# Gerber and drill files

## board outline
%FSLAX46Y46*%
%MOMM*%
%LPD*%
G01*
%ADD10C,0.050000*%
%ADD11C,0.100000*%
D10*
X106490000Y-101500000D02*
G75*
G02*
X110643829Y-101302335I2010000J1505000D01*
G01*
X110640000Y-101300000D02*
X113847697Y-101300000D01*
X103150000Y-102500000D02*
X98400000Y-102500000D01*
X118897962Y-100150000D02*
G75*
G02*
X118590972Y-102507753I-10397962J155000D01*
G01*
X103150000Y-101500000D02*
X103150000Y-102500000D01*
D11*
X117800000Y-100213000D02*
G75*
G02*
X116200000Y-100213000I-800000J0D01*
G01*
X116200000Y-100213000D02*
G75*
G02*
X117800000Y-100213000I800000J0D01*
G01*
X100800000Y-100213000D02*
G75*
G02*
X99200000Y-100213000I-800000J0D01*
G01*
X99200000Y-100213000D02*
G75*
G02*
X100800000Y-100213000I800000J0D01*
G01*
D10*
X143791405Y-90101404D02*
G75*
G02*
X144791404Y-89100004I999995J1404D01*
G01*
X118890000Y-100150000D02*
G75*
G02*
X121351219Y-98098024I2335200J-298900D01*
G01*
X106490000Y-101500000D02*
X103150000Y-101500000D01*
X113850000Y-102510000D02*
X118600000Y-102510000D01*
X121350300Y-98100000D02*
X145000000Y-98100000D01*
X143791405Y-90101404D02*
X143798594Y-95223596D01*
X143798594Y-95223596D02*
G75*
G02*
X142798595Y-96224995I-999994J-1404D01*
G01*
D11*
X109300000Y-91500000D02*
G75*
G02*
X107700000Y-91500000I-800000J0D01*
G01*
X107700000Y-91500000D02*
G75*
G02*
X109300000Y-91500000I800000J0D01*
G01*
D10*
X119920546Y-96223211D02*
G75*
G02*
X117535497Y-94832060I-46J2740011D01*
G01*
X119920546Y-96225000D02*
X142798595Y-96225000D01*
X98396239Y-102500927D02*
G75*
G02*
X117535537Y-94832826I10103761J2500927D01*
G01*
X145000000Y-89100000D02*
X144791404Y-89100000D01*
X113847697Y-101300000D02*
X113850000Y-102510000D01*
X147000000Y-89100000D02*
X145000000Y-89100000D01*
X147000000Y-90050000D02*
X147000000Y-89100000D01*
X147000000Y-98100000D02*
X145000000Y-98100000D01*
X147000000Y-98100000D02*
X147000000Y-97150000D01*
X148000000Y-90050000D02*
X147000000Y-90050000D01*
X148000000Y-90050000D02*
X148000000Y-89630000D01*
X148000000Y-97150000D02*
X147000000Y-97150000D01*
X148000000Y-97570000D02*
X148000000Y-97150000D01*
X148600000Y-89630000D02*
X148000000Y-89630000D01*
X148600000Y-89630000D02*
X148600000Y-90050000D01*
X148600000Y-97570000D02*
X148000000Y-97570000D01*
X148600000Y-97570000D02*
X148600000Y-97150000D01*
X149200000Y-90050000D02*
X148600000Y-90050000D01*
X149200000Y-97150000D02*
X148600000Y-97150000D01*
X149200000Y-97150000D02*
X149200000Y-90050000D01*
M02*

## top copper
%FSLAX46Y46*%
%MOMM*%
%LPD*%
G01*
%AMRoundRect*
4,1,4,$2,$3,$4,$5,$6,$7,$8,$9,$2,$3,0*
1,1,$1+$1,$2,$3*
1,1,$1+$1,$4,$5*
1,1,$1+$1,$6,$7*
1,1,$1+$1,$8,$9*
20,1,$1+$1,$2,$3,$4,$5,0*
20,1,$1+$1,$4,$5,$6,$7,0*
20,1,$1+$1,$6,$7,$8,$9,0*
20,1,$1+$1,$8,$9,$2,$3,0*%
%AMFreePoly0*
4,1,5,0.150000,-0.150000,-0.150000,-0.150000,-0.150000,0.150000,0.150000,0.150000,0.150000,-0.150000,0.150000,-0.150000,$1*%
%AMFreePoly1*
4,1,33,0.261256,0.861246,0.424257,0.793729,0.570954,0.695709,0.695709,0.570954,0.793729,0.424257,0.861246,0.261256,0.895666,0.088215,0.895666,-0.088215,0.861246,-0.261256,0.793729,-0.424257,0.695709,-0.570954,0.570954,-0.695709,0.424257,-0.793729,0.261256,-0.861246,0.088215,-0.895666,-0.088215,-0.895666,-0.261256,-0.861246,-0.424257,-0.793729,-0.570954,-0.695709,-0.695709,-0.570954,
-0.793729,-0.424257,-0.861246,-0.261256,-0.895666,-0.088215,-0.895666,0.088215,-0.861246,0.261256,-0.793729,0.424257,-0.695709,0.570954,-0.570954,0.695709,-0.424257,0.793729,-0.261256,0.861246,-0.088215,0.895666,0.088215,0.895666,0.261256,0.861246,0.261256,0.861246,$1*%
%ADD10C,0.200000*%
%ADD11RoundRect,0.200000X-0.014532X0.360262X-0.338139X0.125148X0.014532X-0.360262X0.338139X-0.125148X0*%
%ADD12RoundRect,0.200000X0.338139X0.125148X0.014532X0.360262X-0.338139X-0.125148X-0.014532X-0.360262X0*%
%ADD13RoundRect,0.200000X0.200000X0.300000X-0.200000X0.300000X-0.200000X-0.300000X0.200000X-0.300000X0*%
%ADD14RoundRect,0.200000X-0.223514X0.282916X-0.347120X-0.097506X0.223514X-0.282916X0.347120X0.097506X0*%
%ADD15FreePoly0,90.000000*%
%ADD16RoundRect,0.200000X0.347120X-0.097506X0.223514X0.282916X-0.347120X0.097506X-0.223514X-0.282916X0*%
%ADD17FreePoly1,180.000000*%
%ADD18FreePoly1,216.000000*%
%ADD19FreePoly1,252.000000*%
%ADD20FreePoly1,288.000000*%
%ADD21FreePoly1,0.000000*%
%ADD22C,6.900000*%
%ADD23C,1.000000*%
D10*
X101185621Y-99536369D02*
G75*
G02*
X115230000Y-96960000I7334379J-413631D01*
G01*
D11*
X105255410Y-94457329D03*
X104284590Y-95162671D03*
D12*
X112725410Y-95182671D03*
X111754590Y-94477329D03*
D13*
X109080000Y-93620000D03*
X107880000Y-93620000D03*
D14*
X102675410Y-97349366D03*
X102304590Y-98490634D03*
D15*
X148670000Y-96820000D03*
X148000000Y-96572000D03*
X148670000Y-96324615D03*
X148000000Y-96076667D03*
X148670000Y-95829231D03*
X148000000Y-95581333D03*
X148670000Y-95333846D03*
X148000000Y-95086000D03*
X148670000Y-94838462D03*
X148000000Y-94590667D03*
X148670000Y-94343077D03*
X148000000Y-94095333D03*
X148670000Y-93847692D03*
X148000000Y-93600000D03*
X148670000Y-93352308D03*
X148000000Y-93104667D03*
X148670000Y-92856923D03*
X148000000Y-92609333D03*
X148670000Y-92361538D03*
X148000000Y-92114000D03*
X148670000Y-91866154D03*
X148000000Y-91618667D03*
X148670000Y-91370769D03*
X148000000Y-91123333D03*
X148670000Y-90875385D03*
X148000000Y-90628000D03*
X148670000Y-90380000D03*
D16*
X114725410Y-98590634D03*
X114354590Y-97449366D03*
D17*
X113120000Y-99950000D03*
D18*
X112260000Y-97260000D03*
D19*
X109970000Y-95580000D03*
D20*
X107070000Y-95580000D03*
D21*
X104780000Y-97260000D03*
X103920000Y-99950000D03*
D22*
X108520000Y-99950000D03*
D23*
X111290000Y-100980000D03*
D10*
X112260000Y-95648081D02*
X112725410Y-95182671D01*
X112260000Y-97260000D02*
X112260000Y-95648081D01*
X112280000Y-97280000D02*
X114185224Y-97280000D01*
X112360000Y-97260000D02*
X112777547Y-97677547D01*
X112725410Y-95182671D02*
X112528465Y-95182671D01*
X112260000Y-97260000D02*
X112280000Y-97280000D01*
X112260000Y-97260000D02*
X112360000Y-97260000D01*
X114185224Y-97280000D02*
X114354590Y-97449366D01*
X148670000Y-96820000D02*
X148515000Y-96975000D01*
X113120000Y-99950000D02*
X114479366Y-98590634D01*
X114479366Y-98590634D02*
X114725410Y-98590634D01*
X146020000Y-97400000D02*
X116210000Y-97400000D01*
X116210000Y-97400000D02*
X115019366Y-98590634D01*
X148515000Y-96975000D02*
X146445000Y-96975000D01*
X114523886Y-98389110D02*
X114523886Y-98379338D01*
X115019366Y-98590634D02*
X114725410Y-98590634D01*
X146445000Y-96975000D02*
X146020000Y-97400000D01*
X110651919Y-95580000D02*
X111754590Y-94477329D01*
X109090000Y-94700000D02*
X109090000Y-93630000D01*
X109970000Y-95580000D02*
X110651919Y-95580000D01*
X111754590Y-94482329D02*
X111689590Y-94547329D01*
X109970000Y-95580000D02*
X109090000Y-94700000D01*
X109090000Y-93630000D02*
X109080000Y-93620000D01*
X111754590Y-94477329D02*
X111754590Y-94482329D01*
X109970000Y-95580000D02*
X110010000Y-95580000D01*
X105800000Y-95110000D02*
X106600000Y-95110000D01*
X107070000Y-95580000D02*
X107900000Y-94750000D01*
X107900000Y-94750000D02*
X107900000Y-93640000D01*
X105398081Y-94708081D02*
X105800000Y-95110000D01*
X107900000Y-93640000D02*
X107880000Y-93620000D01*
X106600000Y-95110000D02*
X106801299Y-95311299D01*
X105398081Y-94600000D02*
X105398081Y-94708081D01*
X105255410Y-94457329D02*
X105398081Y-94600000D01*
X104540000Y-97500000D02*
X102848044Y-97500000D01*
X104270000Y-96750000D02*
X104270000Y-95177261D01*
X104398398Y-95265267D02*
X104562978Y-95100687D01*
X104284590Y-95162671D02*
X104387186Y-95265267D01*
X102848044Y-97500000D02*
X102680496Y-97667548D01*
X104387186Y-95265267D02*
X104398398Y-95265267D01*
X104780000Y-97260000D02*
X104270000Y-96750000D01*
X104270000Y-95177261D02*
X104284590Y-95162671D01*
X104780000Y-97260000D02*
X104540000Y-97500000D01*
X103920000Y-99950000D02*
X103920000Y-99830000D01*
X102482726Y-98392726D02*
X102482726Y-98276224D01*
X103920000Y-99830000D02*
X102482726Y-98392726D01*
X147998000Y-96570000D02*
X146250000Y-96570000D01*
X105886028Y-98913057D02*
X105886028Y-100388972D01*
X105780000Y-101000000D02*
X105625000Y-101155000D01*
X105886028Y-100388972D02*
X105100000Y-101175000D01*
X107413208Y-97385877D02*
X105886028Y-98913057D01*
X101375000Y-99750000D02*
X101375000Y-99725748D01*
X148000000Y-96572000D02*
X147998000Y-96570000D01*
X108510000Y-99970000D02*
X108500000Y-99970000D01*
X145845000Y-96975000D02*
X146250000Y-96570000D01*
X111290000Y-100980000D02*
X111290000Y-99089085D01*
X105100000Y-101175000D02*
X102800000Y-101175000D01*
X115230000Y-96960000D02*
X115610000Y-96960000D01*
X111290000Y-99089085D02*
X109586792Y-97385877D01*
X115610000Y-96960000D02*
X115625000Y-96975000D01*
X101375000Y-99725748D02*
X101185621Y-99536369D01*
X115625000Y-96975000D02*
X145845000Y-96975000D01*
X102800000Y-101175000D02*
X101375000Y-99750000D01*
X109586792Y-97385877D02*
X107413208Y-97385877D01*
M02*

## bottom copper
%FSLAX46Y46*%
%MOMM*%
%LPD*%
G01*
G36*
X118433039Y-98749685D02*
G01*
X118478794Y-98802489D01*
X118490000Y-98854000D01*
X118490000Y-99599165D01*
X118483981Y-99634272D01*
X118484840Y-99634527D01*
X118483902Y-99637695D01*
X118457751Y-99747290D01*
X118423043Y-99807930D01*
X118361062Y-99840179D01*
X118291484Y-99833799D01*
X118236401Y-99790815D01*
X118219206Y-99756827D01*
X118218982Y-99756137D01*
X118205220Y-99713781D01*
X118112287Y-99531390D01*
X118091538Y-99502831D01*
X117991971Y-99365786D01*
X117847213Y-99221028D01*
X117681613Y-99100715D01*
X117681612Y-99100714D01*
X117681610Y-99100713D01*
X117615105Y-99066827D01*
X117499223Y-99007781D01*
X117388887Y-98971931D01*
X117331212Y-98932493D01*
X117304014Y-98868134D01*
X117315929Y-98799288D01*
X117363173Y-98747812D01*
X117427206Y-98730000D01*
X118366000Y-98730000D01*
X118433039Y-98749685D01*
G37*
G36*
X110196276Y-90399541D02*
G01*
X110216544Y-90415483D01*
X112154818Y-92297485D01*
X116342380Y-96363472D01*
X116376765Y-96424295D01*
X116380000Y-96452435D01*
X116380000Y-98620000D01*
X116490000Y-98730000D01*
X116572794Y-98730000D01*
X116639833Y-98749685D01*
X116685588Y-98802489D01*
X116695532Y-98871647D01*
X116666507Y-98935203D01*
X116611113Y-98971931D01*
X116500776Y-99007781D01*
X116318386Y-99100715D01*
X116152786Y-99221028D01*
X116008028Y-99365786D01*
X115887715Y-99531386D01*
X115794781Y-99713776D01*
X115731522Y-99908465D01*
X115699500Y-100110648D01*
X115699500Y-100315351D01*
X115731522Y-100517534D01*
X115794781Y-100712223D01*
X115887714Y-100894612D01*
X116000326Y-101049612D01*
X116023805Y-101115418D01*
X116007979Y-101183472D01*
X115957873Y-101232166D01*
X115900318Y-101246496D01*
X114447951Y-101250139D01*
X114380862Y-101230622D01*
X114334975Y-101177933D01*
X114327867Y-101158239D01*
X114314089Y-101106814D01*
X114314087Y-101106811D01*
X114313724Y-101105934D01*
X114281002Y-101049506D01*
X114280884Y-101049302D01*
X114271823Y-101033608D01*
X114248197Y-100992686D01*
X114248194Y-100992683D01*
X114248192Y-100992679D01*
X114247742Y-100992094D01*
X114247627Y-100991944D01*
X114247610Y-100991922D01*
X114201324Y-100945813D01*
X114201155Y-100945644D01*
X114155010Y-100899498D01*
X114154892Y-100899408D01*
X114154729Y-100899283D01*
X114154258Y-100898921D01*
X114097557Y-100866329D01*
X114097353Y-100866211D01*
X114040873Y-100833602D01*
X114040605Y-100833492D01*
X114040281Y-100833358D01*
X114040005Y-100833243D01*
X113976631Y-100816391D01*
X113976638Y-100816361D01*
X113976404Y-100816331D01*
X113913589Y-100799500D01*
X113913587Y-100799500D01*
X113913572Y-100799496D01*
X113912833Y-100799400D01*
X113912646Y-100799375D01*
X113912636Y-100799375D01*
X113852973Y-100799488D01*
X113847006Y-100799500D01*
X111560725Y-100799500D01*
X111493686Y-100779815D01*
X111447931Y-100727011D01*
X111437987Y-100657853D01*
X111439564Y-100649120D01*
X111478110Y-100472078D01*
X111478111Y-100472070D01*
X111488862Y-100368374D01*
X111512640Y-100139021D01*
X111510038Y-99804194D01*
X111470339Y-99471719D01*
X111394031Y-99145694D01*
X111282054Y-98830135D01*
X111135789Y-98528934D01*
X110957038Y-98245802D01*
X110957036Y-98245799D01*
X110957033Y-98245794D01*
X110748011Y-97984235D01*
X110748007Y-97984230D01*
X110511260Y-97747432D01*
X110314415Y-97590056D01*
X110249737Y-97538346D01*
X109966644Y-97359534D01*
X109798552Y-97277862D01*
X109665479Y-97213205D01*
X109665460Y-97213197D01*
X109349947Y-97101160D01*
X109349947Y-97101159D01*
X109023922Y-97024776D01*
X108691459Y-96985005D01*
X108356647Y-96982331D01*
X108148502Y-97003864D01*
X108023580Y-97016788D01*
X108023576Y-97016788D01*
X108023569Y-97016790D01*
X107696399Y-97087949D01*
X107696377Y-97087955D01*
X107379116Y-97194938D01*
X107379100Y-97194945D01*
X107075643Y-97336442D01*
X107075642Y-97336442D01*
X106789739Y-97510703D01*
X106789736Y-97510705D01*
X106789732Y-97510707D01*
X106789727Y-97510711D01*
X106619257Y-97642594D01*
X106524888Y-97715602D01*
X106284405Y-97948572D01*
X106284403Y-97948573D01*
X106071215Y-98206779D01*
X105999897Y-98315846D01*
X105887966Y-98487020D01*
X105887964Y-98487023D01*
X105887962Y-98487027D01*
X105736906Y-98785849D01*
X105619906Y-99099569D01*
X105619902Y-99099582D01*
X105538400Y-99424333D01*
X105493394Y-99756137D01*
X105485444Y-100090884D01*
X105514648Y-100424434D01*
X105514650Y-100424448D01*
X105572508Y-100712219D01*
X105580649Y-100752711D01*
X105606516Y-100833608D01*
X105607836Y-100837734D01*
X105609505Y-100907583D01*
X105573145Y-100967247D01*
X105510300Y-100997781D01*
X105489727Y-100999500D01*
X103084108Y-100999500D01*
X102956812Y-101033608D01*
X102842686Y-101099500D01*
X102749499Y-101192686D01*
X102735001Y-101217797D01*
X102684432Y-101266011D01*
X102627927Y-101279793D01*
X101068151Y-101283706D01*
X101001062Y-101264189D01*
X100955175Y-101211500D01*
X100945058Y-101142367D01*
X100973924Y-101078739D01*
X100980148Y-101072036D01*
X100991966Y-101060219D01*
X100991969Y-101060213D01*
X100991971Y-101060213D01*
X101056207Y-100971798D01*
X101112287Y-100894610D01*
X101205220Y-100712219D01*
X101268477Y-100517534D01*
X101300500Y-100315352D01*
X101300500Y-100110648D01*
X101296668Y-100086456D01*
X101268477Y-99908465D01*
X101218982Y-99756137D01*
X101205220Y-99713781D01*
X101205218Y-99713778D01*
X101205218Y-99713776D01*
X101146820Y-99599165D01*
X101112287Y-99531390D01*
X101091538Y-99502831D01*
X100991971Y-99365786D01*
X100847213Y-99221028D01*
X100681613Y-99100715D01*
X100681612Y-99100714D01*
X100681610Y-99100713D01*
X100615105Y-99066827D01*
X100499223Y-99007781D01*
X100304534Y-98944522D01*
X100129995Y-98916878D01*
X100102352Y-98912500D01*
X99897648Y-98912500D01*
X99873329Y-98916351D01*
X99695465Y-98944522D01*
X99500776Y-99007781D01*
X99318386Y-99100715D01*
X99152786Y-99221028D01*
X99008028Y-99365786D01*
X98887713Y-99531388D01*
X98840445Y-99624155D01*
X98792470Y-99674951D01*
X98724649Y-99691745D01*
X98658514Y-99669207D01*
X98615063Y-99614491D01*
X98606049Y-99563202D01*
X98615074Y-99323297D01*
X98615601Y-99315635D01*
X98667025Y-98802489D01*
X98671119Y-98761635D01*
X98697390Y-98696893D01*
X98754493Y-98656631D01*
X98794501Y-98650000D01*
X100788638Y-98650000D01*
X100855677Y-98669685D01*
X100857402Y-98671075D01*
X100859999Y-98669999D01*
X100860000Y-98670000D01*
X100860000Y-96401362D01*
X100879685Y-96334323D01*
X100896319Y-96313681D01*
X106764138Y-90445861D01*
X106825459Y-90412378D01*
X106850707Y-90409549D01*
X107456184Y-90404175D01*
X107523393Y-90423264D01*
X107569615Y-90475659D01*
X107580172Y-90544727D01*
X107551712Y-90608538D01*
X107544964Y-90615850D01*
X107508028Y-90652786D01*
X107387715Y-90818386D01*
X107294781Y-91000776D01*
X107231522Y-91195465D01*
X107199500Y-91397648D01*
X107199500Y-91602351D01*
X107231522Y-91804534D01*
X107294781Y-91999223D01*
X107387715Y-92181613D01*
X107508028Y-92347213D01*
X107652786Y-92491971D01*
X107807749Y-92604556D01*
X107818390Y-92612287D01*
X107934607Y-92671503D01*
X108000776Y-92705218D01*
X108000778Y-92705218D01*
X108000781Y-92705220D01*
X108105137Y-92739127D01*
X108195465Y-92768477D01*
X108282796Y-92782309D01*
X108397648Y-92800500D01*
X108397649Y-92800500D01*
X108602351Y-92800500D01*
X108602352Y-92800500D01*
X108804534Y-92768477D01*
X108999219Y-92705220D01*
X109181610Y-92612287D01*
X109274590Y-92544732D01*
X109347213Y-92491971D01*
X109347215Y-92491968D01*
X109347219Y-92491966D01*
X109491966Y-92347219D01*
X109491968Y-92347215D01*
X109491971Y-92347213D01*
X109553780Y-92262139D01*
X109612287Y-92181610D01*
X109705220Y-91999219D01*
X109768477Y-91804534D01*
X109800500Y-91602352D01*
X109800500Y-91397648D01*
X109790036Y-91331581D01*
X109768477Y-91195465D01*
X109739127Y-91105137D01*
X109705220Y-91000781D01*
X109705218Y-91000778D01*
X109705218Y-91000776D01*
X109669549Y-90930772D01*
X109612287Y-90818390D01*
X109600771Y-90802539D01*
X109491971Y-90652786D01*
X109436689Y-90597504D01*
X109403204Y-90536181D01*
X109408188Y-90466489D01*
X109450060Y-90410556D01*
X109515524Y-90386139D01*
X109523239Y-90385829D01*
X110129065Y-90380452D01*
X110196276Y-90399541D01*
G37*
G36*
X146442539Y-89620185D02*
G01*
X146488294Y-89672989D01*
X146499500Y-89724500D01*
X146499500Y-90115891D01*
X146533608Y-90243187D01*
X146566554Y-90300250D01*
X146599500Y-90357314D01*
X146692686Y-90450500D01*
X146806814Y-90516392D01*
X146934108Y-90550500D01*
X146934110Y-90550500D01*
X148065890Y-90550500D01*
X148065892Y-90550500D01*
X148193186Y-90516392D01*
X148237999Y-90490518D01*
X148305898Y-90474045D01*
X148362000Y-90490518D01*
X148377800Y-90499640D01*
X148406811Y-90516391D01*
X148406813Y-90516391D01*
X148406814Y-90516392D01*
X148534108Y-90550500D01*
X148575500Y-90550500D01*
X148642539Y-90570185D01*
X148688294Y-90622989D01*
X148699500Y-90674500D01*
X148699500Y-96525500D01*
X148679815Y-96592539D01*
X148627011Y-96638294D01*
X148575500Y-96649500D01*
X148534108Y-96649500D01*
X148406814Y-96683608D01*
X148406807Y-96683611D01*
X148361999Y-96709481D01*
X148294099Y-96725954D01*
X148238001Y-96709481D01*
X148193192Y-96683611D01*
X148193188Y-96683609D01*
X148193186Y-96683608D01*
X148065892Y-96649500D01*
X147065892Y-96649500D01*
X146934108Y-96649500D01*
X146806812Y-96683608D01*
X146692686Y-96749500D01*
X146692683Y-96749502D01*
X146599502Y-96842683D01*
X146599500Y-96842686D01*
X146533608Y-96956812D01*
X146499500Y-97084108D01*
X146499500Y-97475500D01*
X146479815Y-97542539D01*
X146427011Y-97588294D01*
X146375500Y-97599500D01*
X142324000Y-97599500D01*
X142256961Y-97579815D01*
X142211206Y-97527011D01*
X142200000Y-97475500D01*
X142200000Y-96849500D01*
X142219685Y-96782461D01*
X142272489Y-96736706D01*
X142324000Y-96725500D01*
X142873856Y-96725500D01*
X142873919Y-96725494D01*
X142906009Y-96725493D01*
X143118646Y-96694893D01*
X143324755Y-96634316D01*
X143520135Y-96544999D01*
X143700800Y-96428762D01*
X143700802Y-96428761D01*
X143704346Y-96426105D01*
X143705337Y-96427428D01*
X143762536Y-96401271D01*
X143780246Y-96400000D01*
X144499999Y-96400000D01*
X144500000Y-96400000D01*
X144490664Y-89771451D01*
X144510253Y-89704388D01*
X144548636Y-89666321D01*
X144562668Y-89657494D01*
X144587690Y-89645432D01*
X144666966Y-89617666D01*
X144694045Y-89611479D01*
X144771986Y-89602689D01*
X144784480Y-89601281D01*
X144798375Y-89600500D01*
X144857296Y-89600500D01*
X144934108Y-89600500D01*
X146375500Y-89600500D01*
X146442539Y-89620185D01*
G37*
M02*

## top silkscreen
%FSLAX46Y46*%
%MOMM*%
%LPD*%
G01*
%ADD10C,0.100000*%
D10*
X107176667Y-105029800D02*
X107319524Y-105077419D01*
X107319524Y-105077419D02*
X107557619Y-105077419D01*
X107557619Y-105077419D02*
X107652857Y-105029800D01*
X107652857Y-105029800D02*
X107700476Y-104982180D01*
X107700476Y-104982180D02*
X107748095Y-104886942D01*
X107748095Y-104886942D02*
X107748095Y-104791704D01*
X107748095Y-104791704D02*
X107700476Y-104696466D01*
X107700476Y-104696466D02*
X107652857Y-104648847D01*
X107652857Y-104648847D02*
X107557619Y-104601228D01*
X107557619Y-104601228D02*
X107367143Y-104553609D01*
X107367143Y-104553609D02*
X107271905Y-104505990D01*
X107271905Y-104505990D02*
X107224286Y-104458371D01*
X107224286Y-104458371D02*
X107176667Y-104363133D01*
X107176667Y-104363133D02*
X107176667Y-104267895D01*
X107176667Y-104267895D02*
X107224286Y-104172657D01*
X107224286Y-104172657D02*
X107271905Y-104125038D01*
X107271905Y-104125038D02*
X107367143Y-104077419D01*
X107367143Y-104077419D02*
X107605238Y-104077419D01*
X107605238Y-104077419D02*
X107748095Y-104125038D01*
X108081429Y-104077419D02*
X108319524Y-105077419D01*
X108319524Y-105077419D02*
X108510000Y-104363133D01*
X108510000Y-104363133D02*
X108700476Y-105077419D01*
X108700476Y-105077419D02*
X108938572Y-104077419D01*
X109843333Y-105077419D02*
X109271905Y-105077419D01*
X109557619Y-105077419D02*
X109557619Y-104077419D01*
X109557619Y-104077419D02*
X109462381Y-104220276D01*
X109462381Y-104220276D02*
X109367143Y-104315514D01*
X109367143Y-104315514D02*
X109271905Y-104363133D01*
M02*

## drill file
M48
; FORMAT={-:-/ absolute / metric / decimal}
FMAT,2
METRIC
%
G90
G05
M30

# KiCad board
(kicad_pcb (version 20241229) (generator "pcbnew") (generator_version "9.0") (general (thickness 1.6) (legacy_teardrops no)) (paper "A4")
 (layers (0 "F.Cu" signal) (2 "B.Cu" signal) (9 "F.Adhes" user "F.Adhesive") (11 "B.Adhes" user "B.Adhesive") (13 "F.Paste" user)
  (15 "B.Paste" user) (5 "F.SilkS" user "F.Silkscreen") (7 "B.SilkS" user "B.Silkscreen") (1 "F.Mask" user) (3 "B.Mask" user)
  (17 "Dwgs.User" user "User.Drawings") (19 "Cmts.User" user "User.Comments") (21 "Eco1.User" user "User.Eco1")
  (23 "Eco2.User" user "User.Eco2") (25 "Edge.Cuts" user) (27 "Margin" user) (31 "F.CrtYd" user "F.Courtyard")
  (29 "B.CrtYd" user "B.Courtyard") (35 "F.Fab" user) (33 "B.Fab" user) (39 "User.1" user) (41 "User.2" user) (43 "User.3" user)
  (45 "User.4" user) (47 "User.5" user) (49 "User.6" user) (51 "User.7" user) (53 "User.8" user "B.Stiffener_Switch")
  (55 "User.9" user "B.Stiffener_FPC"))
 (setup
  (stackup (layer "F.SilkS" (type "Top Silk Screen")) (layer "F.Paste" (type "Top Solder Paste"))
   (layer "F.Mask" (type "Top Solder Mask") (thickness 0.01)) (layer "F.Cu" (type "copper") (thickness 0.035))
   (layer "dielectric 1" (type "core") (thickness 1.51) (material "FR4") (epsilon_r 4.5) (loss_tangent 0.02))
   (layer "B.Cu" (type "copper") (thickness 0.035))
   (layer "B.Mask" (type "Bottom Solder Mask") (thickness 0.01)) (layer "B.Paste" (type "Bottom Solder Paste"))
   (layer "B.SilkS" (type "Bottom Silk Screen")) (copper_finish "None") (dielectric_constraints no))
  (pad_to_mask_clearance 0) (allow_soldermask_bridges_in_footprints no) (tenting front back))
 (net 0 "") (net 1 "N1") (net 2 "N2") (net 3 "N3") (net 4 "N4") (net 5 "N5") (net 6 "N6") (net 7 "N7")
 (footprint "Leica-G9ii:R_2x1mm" (layer "F.Cu") (at 104.77 94.81 -144)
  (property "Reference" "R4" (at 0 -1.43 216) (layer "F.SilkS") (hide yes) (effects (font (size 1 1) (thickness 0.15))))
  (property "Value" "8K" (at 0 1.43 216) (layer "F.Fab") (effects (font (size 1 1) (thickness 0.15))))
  (pad "" smd roundrect (at -0.6 0 216) (size 0.6 0.8) (layers "F.Mask" "F.Paste") (roundrect_rratio 0.25))
  (pad "" smd roundrect (at 0.61 0 216) (size 0.6 0.8) (layers "F.Mask" "F.Paste") (roundrect_rratio 0.25))
  (pad "1" smd roundrect (at -0.6 0 216) (size 0.8 1) (layers "F.Cu") (roundrect_rratio 0.25) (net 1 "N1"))
  (pad "2" smd roundrect (at 0.6 0 216) (size 0.8 1) (layers "F.Cu") (roundrect_rratio 0.25) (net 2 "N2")))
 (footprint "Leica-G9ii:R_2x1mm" (layer "F.Cu") (at 112.24 94.83 144)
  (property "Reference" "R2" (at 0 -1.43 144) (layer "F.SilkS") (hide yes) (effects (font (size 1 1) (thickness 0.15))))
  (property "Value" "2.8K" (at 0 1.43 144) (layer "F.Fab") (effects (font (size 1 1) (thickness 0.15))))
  (pad "" smd roundrect (at -0.6 0 144) (size 0.6 0.8) (layers "F.Mask" "F.Paste") (roundrect_rratio 0.25))
  (pad "" smd roundrect (at 0.61 0 144) (size 0.6 0.8) (layers "F.Mask" "F.Paste") (roundrect_rratio 0.25))
  (pad "1" smd roundrect (at -0.6 0 144) (size 0.8 1) (layers "F.Cu") (roundrect_rratio 0.25) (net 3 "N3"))
  (pad "2" smd roundrect (at 0.6 0 144) (size 0.8 1) (layers "F.Cu") (roundrect_rratio 0.25) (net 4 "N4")))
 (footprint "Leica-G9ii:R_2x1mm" (layer "F.Cu") (at 108.48 93.62 180)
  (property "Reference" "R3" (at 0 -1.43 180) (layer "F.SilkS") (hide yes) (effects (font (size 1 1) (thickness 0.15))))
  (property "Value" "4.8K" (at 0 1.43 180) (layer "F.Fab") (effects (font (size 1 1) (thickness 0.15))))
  (pad "" smd roundrect (at -0.6 0 180) (size 0.6 0.8) (layers "F.Mask" "F.Paste") (roundrect_rratio 0.25))
  (pad "" smd roundrect (at 0.61 0 180) (size 0.6 0.8) (layers "F.Mask" "F.Paste") (roundrect_rratio 0.25))
  (pad "1" smd roundrect (at -0.6 0 180) (size 0.8 1) (layers "F.Cu") (roundrect_rratio 0.25) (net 4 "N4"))
  (pad "2" smd roundrect (at 0.6 0 180) (size 0.8 1) (layers "F.Cu") (roundrect_rratio 0.25) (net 1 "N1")))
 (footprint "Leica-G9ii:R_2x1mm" (layer "F.Cu") (at 102.49 97.92 -108)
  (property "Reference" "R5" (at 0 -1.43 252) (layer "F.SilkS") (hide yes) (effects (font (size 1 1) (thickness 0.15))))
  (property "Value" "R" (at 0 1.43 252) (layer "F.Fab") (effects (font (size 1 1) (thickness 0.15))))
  (pad "" smd roundrect (at -0.6 0 252) (size 0.6 0.8) (layers "F.Mask" "F.Paste") (roundrect_rratio 0.25))
  (pad "" smd roundrect (at 0.609999 0 252) (size 0.6 0.8) (layers "F.Mask" "F.Paste") (roundrect_rratio 0.25))
  (pad "1" smd roundrect (at -0.6 0 252) (size 0.8 1) (layers "F.Cu") (roundrect_rratio 0.25) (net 2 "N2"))
  (pad "2" smd roundrect (at 0.6 0 252) (size 0.8 1) (layers "F.Cu") (roundrect_rratio 0.25) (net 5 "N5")))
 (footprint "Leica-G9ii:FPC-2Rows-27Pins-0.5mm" (layer "F.Cu") (at 147 93.6 90)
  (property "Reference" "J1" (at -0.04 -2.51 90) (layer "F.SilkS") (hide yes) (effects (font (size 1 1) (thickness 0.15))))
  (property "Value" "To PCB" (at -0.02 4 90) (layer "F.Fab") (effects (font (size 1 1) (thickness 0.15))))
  (fp_line (start 4.5 0) (end 4.5 -2) (stroke (width 0.05) (type solid)) (layer "Edge.Cuts"))
  (fp_line (start 3.55 0) (end 4.5 0) (stroke (width 0.05) (type solid)) (layer "Edge.Cuts"))
  (fp_line (start -4.5 0) (end -4.5 -2) (stroke (width 0.05) (type solid)) (layer "Edge.Cuts"))
  (fp_line (start -4.5 0) (end -3.55 0) (stroke (width 0.05) (type solid)) (layer "Edge.Cuts"))
  (fp_line (start 3.55 1) (end 3.55 0) (stroke (width 0.05) (type solid)) (layer "Edge.Cuts"))
  (fp_line (start 3.55 1) (end 3.97 1) (stroke (width 0.05) (type default)) (layer "Edge.Cuts"))
  (fp_line (start -3.55 1) (end -3.55 0) (stroke (width 0.05) (type solid)) (layer "Edge.Cuts"))
  (fp_line (start -3.97 1) (end -3.55 1) (stroke (width 0.05) (type default)) (layer "Edge.Cuts"))
  (fp_line (start 3.97 1.6) (end 3.97 1) (stroke (width 0.05) (type solid)) (layer "Edge.Cuts"))
  (fp_line (start 3.97 1.6) (end 3.55 1.6) (stroke (width 0.05) (type default)) (layer "Edge.Cuts"))
  (fp_line (start -3.97 1.6) (end -3.97 1) (stroke (width 0.05) (type solid)) (layer "Edge.Cuts"))
  (fp_line (start -3.97 1.6) (end -3.55 1.6) (stroke (width 0.05) (type default)) (layer "Edge.Cuts"))
  (fp_line (start 3.55 2.2) (end 3.55 1.6) (stroke (width 0.05) (type solid)) (layer "Edge.Cuts"))
  (fp_line (start -3.55 2.2) (end -3.55 1.6) (stroke (width 0.05) (type solid)) (layer "Edge.Cuts"))
  (fp_line (start -3.55 2.2) (end 3.55 2.2) (stroke (width 0.05) (type solid)) (layer "Edge.Cuts"))
  (pad "1" smd custom (at -3.22 1.67 90) (size 0.3 0.3) (layers "F.Cu" "F.Mask" "F.Paste") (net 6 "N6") (clearance 0.07)
   (options (clearance outline) (anchor rect)) (primitives))
  (pad "2" smd custom (at -2.972 1 90) (size 0.3 0.3) (layers "F.Cu" "F.Mask" "F.Paste") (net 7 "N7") (clearance 0.07)
   (options (clearance outline) (anchor rect)) (primitives))
  (pad "3" smd custom (at -2.724615 1.67 90) (size 0.3 0.3) (layers "F.Cu" "F.Mask" "F.Paste") (clearance 0.07)
   (options (clearance outline) (anchor rect)) (primitives))
  (pad "4" smd custom (at -2.476667 1 90) (size 0.3 0.3) (layers "F.Cu" "F.Mask" "F.Paste") (clearance 0.07)
   (options (clearance outline) (anchor rect)) (primitives))
  (pad "5" smd custom (at -2.229231 1.67 90) (size 0.3 0.3) (layers "F.Cu" "F.Mask" "F.Paste") (options (clearance outline) (anchor rect))
   (primitives))
  (pad "6" smd custom (at -1.981333 1 90) (size 0.3 0.3) (layers "F.Cu" "F.Mask" "F.Paste") (clearance 0.1)
   (options (clearance outline) (anchor rect)) (primitives))
  (pad "7" smd custom (at -1.733846 1.67 90) (size 0.3 0.3) (layers "F.Cu" "F.Mask" "F.Paste") (options (clearance outline) (anchor rect))
   (primitives))
  (pad "8" smd custom (at -1.486 1 90) (size 0.3 0.3) (layers "F.Cu" "F.Mask" "F.Paste") (clearance 0.1)
   (options (clearance outline) (anchor rect)) (primitives))
  (pad "9" smd custom (at -1.238462 1.67 90) (size 0.3 0.3) (layers "F.Cu" "F.Mask" "F.Paste") (options (clearance outline) (anchor rect))
   (primitives))
  (pad "10" smd custom (at -0.990667 1 90) (size 0.3 0.3) (layers "F.Cu" "F.Mask" "F.Paste") (clearance 0.1)
   (options (clearance outline) (anchor rect)) (primitives))
  (pad "11" smd custom (at -0.743077 1.67 90) (size 0.3 0.3) (layers "F.Cu" "F.Mask" "F.Paste") (options (clearance outline) (anchor rect))
   (primitives))
  (pad "12" smd custom (at -0.495333 1 90) (size 0.3 0.3) (layers "F.Cu" "F.Mask" "F.Paste") (clearance 0.1)
   (options (clearance outline) (anchor rect)) (primitives))
  (pad "13" smd custom (at -0.247692 1.67 90) (size 0.3 0.3) (layers "F.Cu" "F.Mask" "F.Paste") (options (clearance outline) (anchor rect))
   (primitives))
  (pad "14" smd custom (at 0 1 90) (size 0.3 0.3) (layers "F.Cu" "F.Mask" "F.Paste") (clearance 0.1)
   (options (clearance outline) (anchor rect)) (primitives))
  (pad "15" smd custom (at 0.247692 1.67 90) (size 0.3 0.3) (layers "F.Cu" "F.Mask" "F.Paste") (options (clearance outline) (anchor rect))
   (primitives))
  (pad "16" smd custom (at 0.495333 1 90) (size 0.3 0.3) (layers "F.Cu" "F.Mask" "F.Paste") (clearance 0.1)
   (options (clearance outline) (anchor rect)) (primitives))
  (pad "17" smd custom (at 0.743077 1.67 90) (size 0.3 0.3) (layers "F.Cu" "F.Mask" "F.Paste") (options (clearance outline) (anchor rect))
   (primitives))
  (pad "18" smd custom (at 0.990667 1 90) (size 0.3 0.3) (layers "F.Cu" "F.Mask" "F.Paste") (clearance 0.1)
   (options (clearance outline) (anchor rect)) (primitives))
  (pad "19" smd custom (at 1.238462 1.67 90) (size 0.3 0.3) (layers "F.Cu" "F.Mask" "F.Paste") (options (clearance outline) (anchor rect))
   (primitives))
  (pad "20" smd custom (at 1.486 1 90) (size 0.3 0.3) (layers "F.Cu" "F.Mask" "F.Paste") (clearance 0.1)
   (options (clearance outline) (anchor rect)) (primitives))
  (pad "21" smd custom (at 1.733846 1.67 90) (size 0.3 0.3) (layers "F.Cu" "F.Mask" "F.Paste") (options (clearance outline) (anchor rect))
   (primitives))
  (pad "22" smd custom (at 1.981333 1 90) (size 0.3 0.3) (layers "F.Cu" "F.Mask" "F.Paste") (clearance 0.1)
   (options (clearance outline) (anchor rect)) (primitives))
  (pad "23" smd custom (at 2.229231 1.67 90) (size 0.3 0.3) (layers "F.Cu" "F.Mask" "F.Paste") (options (clearance outline) (anchor rect))
   (primitives))
  (pad "24" smd custom (at 2.476667 1 90) (size 0.3 0.3) (layers "F.Cu" "F.Mask" "F.Paste") (clearance 0.1)
   (options (clearance outline) (anchor rect)) (primitives))
  (pad "25" smd custom (at 2.724615 1.67 90) (size 0.3 0.3) (layers "F.Cu" "F.Mask" "F.Paste") (options (clearance outline) (anchor rect))
   (primitives))
  (pad "26" smd custom (at 2.972 1 90) (size 0.3 0.3) (layers "F.Cu" "F.Mask" "F.Paste") (clearance 0.1)
   (options (clearance outline) (anchor rect)) (primitives))
  (pad "27" smd custom (at 3.22 1.67 90) (size 0.3 0.3) (layers "F.Cu" "F.Mask" "F.Paste") (options (clearance outline) (anchor rect))
   (primitives)))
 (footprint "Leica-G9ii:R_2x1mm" (layer "F.Cu") (at 114.54 98.02 108)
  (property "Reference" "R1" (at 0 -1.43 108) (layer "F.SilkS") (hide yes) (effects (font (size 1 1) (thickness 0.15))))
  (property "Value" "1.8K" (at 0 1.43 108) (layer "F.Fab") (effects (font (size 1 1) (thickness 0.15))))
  (pad "" smd roundrect (at -0.6 0 108) (size 0.6 0.8) (layers "F.Mask" "F.Paste") (roundrect_rratio 0.25))
  (pad "" smd roundrect (at 0.609999 0 108) (size 0.6 0.8) (layers "F.Mask" "F.Paste") (roundrect_rratio 0.25))
  (pad "1" smd roundrect (at -0.6 0 108) (size 0.8 1) (layers "F.Cu") (roundrect_rratio 0.25) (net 6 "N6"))
  (pad "2" smd roundrect (at 0.6 0 108) (size 0.8 1) (layers "F.Cu") (roundrect_rratio 0.25) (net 3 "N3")))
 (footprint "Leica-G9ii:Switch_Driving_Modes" (layer "F.Cu") (at 108.52 99.95)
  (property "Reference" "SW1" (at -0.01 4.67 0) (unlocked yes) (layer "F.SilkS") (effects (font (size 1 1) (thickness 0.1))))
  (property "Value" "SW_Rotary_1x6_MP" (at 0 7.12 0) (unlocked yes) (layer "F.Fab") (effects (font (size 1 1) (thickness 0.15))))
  (pad "1" smd custom (at 4.6 0 180) (size 1.8 1.8) (layers "F.Cu" "F.Mask" "F.Paste") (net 6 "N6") (clearance 0.14)
   (thermal_bridge_angle 90) (options (clearance outline) (anchor circle)) (primitives))
  (pad "2" smd custom (at 3.74 -2.69 216) (size 1.8 1.8) (layers "F.Cu" "F.Mask" "F.Paste") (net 3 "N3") (clearance 0.14)
   (thermal_bridge_angle 90) (options (clearance outline) (anchor circle)) (primitives))
  (pad "3" smd custom (at 1.45 -4.37 252) (size 1.8 1.8) (layers "F.Cu" "F.Mask" "F.Paste") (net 4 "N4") (clearance 0.14)
   (thermal_bridge_angle 90) (options (clearance outline) (anchor circle)) (primitives))
  (pad "4" smd custom (at -1.45 -4.37 288) (size 1.8 1.8) (layers "F.Cu" "F.Mask" "F.Paste") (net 1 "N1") (clearance 0.14)
   (thermal_bridge_angle 90) (options (clearance outline) (anchor circle)) (primitives))
  (pad "5" smd custom (at -3.74 -2.69) (size 1.8 1.8) (layers "F.Cu" "F.Mask" "F.Paste") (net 2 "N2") (clearance 0.14)
   (options (clearance outline) (anchor circle)) (primitives))
  (pad "6" smd custom (at -4.6 0) (size 1.8 1.8) (layers "F.Cu" "F.Mask" "F.Paste") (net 5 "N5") (clearance 0.14) (thermal_bridge_angle 90)
   (options (clearance outline) (anchor circle)) (primitives))
  (pad "7" smd circle (at 0 0) (size 6.9 6.9) (layers "F.Cu" "F.Mask" "F.Paste") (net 7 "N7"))
  (pad "7" smd circle (at 2.77 1.03) (size 1 1) (layers "F.Cu" "F.Mask" "F.Paste") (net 7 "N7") (clearance 0.1)))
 (gr_arc (start 101.185621 99.536369) (mid 107.194526 92.724536) (end 115.23 96.96) (stroke (width 0.2) (type default)) (layer "F.Cu")
  (net 7))
 (gr_arc (start 106.49 101.5) (mid 108.380646 97.486841) (end 110.643829 101.302335) (stroke (width 0.05) (type default))
  (layer "Edge.Cuts"))
 (gr_line (start 110.64 101.3) (end 113.847697 101.3) (stroke (width 0.05) (type default)) (layer "Edge.Cuts"))
 (gr_line (start 103.15 102.5) (end 98.4 102.5) (stroke (width 0.05) (type default)) (layer "Edge.Cuts"))
 (gr_arc (start 118.897962 100.15) (mid 118.812073 101.337679) (end 118.590972 102.507753) (stroke (width 0.05) (type default))
  (layer "Edge.Cuts"))
 (gr_line (start 103.15 101.5) (end 103.15 102.5) (stroke (width 0.05) (type default)) (layer "Edge.Cuts"))
 (gr_circle (center 117 100.213) (end 117.8 100.213) (stroke (width 0.1) (type default)) (fill no) (layer "Edge.Cuts"))
 (gr_circle (center 100 100.213) (end 100.8 100.213) (stroke (width 0.1) (type default)) (fill no) (layer "Edge.Cuts"))
 (gr_arc (start 143.791405 90.101404) (mid 144.083801 89.39339) (end 144.791404 89.1) (stroke (width 0.05) (type default))
  (layer "Edge.Cuts"))
 (gr_arc (start 118.89 100.15) (mid 119.717627 98.640646) (end 121.351221 98.097981) (stroke (width 0.05) (type default))
  (layer "Edge.Cuts"))
 (gr_line (start 106.49 101.5) (end 103.15 101.5) (stroke (width 0.05) (type solid)) (layer "Edge.Cuts"))
 (gr_line (start 113.85 102.51) (end 118.6 102.51) (stroke (width 0.05) (type default)) (layer "Edge.Cuts"))
 (gr_line (start 121.3503 98.1) (end 145 98.1) (stroke (width 0.05) (type default)) (layer "Edge.Cuts"))
 (gr_line (start 143.791405 90.101404) (end 143.798594 95.223596) (stroke (width 0.05) (type default)) (layer "Edge.Cuts"))
 (gr_arc (start 143.798594 95.223596) (mid 143.506198 95.93161) (end 142.798595 96.225) (stroke (width 0.05) (type default))
  (layer "Edge.Cuts"))
 (gr_circle (center 108.5 91.5) (end 109.3 91.5) (stroke (width 0.1) (type default)) (fill no) (layer "Edge.Cuts"))
 (gr_arc (start 119.920546 96.223211) (mid 118.54 95.85) (end 117.535537 94.832037) (stroke (width 0.05) (type default)) (layer "Edge.Cuts"))
 (gr_line (start 119.920546 96.225) (end 142.798595 96.225) (stroke (width 0.05) (type default)) (layer "Edge.Cuts"))
 (gr_arc (start 98.396239 102.500927) (mid 104.628925 90.33794) (end 117.535537 94.832826) (stroke (width 0.05) (type default))
  (layer "Edge.Cuts"))
 (gr_line (start 145 89.1) (end 144.791404 89.1) (stroke (width 0.05) (type default)) (layer "Edge.Cuts"))
 (gr_line (start 113.847697 101.3) (end 113.85 102.51) (stroke (width 0.05) (type default)) (layer "Edge.Cuts"))
 (segment (start 112.26 95.648081) (end 112.72541 95.182671) (width 0.2) (layer "F.Cu") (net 3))
 (segment (start 112.26 97.26) (end 112.26 95.648081) (width 0.2) (layer "F.Cu") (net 3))
 (segment (start 112.28 97.28) (end 114.185224 97.28) (width 0.2) (layer "F.Cu") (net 3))
 (segment (start 112.36 97.26) (end 112.777547 97.677547) (width 0.2) (layer "F.Cu") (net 3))
 (segment (start 112.72541 95.182671) (end 112.528465 95.182671) (width 0.2) (layer "F.Cu") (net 3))
 (segment (start 112.26 97.26) (end 112.28 97.28) (width 0.2) (layer "F.Cu") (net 3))
 (segment (start 112.26 97.26) (end 112.36 97.26) (width 0.2) (layer "F.Cu") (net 3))
 (segment (start 114.185224 97.28) (end 114.35459 97.449366) (width 0.2) (layer "F.Cu") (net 3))
 (segment (start 148.67 96.82) (end 148.515 96.975) (width 0.2) (layer "F.Cu") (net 6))
 (segment (start 113.12 99.95) (end 114.479366 98.590634) (width 0.2) (layer "F.Cu") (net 6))
 (segment (start 114.479366 98.590634) (end 114.72541 98.590634) (width 0.2) (layer "F.Cu") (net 6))
 (segment (start 146.02 97.4) (end 116.21 97.4) (width 0.2) (layer "F.Cu") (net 6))
 (segment (start 116.21 97.4) (end 115.019366 98.590634) (width 0.2) (layer "F.Cu") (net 6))
 (segment (start 148.515 96.975) (end 146.445 96.975) (width 0.2) (layer "F.Cu") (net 6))
 (segment (start 114.523886 98.38911) (end 114.523886 98.379338) (width 0.2) (layer "F.Cu") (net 6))
 (segment (start 115.019366 98.590634) (end 114.72541 98.590634) (width 0.2) (layer "F.Cu") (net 6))
 (segment (start 146.445 96.975) (end 146.02 97.4) (width 0.2) (layer "F.Cu") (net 6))
 (segment (start 110.651919 95.58) (end 111.75459 94.477329) (width 0.2) (layer "F.Cu") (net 4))
 (segment (start 109.09 94.7) (end 109.09 93.63) (width 0.2) (layer "F.Cu") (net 4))
 (segment (start 109.97 95.58) (end 110.651919 95.58) (width 0.2) (layer "F.Cu") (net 4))
 (segment (start 111.75459 94.482329) (end 111.68959 94.547329) (width 0.2) (layer "F.Cu") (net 4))
 (segment (start 109.97 95.58) (end 109.09 94.7) (width 0.2) (layer "F.Cu") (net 4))
 (segment (start 109.09 93.63) (end 109.08 93.62) (width 0.2) (layer "F.Cu") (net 4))
 (segment (start 111.75459 94.477329) (end 111.75459 94.482329) (width 0.2) (layer "F.Cu") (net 4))
 (segment (start 109.97 95.58) (end 110.01 95.58) (width 0.2) (layer "F.Cu") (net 4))
 (segment (start 105.8 95.11) (end 106.6 95.11) (width 0.2) (layer "F.Cu") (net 1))
 (segment (start 107.07 95.58) (end 107.9 94.75) (width 0.2) (layer "F.Cu") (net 1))
 (segment (start 107.9 94.75) (end 107.9 93.64) (width 0.2) (layer "F.Cu") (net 1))
 (segment (start 105.398081 94.708081) (end 105.8 95.11) (width 0.2) (layer "F.Cu") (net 1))
 (segment (start 107.9 93.64) (end 107.88 93.62) (width 0.2) (layer "F.Cu") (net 1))
 (segment (start 106.6 95.11) (end 106.801299 95.311299) (width 0.2) (layer "F.Cu") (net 1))
 (segment (start 105.398081 94.6) (end 105.398081 94.708081) (width 0.2) (layer "F.Cu") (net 1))
 (segment (start 105.25541 94.457329) (end 105.398081 94.6) (width 0.2) (layer "F.Cu") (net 1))
 (segment (start 104.54 97.5) (end 102.848044 97.5) (width 0.2) (layer "F.Cu") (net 2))
 (segment (start 104.27 96.75) (end 104.27 95.177261) (width 0.2) (layer "F.Cu") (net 2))
 (segment (start 104.398398 95.265267) (end 104.562978 95.100687) (width 0.2) (layer "F.Cu") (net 2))
 (segment (start 104.28459 95.162671) (end 104.387186 95.265267) (width 0.2) (layer "F.Cu") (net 2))
 (segment (start 102.848044 97.5) (end 102.680496 97.667548) (width 0.2) (layer "F.Cu") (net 2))
 (segment (start 104.387186 95.265267) (end 104.398398 95.265267) (width 0.2) (layer "F.Cu") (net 2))
 (segment (start 104.78 97.26) (end 104.27 96.75) (width 0.2) (layer "F.Cu") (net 2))
 (segment (start 104.27 95.177261) (end 104.28459 95.162671) (width 0.2) (layer "F.Cu") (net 2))
 (segment (start 104.78 97.26) (end 104.54 97.5) (width 0.2) (layer "F.Cu") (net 2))
 (segment (start 103.92 99.95) (end 103.92 99.83) (width 0.2) (layer "F.Cu") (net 5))
 (segment (start 102.482726 98.392726) (end 102.482726 98.276224) (width 0.2) (layer "F.Cu") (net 5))
 (segment (start 103.92 99.83) (end 102.482726 98.392726) (width 0.2) (layer "F.Cu") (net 5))
 (segment (start 147.998 96.57) (end 146.25 96.57) (width 0.2) (layer "F.Cu") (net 7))
 (segment (start 105.886028 98.913057) (end 105.886028 100.388972) (width 0.2) (layer "F.Cu") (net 7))
 (segment (start 105.78 101) (end 105.625 101.155) (width 0.2) (layer "F.Cu") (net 7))
 (segment (start 105.886028 100.388972) (end 105.1 101.175) (width 0.2) (layer "F.Cu") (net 7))
 (segment (start 107.413208 97.385877) (end 105.886028 98.913057) (width 0.2) (layer "F.Cu") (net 7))
 (segment (start 101.375 99.75) (end 101.375 99.725748) (width 0.2) (layer "F.Cu") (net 7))
 (segment (start 148 96.572) (end 147.998 96.57) (width 0.2) (layer "F.Cu") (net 7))
 (segment (start 108.51 99.97) (end 108.5 99.97) (width 0.2) (layer "F.Cu") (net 7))
 (segment (start 145.845 96.975) (end 146.25 96.57) (width 0.2) (layer "F.Cu") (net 7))
 (segment (start 111.29 100.98) (end 111.29 99.089085) (width 0.2) (layer "F.Cu") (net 7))
 (segment (start 105.1 101.175) (end 102.8 101.175) (width 0.2) (layer "F.Cu") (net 7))
 (segment (start 115.23 96.96) (end 115.61 96.96) (width 0.2) (layer "F.Cu") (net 7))
 (segment (start 111.29 99.089085) (end 109.586792 97.385877) (width 0.2) (layer "F.Cu") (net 7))
 (segment (start 115.61 96.96) (end 115.625 96.975) (width 0.2) (layer "F.Cu") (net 7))
 (segment (start 101.375 99.725748) (end 101.185621 99.536369) (width 0.2) (layer "F.Cu") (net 7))
 (segment (start 115.625 96.975) (end 145.845 96.975) (width 0.2) (layer "F.Cu") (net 7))
 (segment (start 102.8 101.175) (end 101.375 99.75) (width 0.2) (layer "F.Cu") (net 7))
 (segment (start 109.586792 97.385877) (end 107.413208 97.385877) (width 0.2) (layer "F.Cu") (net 7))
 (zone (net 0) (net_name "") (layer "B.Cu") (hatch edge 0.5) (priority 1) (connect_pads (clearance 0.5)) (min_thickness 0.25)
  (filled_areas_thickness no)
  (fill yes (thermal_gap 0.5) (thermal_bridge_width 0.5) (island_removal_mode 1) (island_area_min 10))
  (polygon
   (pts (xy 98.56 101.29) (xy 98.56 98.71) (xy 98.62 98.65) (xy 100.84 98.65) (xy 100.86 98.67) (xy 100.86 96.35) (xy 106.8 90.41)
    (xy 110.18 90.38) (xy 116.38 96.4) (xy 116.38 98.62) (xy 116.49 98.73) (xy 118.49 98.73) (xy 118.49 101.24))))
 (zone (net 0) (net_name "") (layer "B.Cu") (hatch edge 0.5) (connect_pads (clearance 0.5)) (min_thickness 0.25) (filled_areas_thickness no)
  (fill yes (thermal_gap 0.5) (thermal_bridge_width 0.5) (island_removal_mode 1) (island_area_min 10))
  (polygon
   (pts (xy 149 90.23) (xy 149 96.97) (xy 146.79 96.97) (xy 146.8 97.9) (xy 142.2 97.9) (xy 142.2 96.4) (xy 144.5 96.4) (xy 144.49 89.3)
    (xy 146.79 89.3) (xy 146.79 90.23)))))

